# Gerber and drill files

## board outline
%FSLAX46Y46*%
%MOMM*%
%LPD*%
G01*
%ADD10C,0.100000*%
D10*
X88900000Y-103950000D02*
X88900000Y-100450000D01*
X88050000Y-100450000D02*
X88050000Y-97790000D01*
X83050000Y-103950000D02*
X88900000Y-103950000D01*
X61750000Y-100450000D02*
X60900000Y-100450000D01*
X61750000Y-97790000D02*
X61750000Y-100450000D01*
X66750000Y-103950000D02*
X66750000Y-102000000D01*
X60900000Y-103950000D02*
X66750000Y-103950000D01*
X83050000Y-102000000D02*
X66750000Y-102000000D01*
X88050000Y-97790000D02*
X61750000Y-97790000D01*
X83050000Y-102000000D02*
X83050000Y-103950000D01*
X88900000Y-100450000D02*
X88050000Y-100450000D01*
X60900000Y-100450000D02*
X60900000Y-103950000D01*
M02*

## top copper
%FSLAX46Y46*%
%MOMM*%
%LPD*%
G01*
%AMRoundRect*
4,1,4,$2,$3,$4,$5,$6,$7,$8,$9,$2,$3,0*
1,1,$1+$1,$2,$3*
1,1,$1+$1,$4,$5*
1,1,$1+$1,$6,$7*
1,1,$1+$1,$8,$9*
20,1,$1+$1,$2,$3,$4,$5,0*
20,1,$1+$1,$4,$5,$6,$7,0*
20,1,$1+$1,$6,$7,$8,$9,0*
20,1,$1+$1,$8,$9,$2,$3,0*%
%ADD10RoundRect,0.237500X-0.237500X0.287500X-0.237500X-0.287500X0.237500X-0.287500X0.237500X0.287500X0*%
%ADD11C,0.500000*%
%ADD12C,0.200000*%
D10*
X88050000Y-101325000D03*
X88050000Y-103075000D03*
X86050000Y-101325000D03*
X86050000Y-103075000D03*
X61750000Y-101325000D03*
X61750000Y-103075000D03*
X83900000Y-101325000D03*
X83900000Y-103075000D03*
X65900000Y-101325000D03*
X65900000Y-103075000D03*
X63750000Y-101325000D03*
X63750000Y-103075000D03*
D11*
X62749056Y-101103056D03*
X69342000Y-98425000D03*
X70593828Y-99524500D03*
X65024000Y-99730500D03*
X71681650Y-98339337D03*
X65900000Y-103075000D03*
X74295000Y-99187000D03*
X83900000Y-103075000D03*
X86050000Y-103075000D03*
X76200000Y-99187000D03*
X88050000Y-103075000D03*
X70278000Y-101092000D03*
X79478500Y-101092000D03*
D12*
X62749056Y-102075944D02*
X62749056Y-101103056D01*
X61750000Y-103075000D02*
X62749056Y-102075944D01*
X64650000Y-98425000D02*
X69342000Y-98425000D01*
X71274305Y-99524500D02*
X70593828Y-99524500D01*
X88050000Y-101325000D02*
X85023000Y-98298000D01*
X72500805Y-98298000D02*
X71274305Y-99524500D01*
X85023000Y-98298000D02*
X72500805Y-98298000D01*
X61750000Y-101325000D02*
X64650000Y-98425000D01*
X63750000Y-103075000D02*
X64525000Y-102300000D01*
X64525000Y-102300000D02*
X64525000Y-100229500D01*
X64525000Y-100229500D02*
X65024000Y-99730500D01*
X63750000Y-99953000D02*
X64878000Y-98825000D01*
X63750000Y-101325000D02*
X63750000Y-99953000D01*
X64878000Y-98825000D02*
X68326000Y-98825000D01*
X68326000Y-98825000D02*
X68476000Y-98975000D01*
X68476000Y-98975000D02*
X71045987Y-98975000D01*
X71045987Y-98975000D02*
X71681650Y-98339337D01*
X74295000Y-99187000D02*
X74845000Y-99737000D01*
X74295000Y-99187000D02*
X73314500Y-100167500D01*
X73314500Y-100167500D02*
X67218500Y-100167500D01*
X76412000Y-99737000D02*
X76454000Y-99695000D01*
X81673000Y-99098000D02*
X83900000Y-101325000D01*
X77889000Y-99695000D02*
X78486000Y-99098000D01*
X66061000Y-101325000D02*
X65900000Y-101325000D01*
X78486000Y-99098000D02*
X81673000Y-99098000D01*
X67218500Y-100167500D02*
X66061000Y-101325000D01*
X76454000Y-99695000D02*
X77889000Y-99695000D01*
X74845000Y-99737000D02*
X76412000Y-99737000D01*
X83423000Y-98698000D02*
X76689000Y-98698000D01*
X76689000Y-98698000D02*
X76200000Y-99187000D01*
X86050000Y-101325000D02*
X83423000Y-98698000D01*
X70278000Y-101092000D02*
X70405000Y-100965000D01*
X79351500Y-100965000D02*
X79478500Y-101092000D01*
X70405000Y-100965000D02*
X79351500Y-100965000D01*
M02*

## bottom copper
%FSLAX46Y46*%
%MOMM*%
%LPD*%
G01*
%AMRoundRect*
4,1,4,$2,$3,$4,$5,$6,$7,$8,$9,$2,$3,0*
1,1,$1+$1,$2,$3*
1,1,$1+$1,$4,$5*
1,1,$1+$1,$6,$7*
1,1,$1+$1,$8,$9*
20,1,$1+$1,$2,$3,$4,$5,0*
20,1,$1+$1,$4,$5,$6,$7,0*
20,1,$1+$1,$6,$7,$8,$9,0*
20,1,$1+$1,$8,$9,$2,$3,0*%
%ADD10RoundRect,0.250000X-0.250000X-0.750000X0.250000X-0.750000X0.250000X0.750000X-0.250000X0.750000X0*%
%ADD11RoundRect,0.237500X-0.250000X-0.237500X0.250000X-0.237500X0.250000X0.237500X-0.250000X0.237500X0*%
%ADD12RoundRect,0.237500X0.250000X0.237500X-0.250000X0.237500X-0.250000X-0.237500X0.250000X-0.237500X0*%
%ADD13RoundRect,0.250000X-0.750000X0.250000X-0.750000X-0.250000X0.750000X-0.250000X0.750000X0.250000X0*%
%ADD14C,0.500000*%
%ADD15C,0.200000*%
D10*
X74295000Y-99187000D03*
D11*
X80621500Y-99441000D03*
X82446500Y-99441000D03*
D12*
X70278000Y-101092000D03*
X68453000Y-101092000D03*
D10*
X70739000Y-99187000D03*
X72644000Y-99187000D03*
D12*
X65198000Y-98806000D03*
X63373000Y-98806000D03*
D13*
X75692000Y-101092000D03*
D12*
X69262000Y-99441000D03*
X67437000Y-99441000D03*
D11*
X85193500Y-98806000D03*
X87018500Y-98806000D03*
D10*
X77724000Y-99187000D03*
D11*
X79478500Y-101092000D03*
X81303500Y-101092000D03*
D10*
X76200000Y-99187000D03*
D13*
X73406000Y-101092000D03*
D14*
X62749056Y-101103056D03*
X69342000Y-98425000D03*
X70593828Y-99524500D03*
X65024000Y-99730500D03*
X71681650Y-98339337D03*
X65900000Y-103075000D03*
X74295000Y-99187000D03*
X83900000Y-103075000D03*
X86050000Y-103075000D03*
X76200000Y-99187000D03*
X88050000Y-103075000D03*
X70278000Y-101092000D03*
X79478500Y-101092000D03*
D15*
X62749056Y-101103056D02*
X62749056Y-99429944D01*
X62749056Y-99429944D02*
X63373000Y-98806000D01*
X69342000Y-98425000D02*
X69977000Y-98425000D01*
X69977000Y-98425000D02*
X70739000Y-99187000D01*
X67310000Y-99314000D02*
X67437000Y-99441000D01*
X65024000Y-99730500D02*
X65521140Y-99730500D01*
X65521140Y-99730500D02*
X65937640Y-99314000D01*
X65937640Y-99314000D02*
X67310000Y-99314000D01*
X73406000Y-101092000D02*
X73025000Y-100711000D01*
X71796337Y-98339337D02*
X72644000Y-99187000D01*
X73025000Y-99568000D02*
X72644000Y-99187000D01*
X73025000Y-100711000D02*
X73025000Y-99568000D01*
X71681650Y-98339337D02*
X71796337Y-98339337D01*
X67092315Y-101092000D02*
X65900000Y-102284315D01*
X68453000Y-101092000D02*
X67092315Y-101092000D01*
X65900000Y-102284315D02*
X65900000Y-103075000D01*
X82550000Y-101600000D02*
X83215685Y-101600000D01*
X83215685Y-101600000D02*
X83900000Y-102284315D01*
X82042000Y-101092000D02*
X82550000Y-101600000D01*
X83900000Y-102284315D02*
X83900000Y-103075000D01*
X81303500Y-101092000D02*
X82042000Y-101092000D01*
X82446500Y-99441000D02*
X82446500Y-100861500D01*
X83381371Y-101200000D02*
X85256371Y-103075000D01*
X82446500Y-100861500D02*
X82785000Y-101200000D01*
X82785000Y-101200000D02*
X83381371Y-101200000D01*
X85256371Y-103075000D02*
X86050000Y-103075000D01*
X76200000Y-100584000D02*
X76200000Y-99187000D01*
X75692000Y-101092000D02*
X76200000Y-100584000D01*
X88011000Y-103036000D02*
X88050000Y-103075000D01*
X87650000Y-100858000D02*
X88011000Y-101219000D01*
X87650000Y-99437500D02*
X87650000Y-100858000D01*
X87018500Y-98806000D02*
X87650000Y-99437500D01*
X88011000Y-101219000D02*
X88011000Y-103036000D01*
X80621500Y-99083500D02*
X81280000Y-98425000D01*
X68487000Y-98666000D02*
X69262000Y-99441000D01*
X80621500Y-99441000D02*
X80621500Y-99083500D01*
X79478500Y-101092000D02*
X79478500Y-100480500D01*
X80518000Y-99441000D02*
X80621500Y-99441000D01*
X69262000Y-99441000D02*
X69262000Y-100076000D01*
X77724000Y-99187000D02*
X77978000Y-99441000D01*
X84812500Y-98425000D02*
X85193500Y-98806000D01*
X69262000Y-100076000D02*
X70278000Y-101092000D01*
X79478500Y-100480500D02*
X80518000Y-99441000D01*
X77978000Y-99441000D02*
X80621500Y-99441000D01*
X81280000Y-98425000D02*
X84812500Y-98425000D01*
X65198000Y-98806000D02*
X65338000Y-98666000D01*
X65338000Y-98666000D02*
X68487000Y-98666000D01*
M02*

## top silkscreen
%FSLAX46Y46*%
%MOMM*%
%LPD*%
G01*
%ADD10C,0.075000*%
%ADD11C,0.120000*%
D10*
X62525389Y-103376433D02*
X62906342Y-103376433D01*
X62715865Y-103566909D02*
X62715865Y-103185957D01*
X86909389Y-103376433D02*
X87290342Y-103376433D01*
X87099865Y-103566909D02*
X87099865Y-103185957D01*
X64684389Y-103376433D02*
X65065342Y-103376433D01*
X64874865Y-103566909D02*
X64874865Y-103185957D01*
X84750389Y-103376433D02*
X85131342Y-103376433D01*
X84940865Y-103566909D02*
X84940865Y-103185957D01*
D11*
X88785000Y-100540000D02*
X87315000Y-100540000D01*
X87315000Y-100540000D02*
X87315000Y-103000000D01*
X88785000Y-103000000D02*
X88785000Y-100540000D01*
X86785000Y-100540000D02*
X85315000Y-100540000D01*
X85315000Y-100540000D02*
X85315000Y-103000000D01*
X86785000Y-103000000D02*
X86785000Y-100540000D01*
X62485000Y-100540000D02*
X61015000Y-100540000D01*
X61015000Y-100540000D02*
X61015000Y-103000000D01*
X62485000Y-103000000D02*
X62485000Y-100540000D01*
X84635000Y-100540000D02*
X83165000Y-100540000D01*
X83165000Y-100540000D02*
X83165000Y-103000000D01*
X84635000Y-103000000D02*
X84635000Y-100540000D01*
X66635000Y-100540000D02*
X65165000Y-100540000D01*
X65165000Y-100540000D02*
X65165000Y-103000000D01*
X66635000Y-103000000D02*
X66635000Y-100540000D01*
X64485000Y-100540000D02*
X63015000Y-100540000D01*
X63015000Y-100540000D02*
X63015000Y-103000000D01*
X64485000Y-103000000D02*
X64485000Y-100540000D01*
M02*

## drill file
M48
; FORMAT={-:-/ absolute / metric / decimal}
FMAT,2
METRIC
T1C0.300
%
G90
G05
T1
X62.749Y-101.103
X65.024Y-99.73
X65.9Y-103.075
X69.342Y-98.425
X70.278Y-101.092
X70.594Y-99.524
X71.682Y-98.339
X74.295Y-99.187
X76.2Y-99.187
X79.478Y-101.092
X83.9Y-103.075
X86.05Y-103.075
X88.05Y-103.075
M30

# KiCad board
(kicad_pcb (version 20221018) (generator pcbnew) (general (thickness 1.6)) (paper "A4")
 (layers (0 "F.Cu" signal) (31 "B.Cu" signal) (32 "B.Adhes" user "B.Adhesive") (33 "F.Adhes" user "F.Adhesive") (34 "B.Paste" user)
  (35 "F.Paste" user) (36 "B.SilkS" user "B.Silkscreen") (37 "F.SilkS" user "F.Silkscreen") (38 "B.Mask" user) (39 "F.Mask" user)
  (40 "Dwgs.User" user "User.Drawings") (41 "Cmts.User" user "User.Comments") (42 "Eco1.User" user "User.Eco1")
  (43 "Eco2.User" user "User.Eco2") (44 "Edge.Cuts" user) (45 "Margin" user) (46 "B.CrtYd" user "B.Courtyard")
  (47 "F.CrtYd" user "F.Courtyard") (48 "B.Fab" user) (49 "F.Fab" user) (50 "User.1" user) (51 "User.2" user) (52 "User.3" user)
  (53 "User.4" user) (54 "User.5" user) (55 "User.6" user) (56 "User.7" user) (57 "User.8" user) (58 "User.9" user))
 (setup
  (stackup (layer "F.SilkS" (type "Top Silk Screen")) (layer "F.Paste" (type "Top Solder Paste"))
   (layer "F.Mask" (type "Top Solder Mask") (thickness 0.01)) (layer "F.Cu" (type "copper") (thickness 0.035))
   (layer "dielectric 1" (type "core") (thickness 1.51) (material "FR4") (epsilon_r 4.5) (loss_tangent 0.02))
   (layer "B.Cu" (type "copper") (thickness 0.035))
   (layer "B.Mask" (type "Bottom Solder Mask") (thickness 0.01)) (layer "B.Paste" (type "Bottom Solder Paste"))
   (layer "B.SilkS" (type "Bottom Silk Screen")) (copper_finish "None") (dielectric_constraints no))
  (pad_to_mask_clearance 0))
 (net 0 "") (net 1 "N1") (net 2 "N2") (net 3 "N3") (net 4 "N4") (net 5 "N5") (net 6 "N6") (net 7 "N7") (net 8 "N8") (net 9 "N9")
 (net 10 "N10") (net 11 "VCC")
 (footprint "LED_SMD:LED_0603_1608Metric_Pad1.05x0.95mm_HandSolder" (layer "F.Cu") (at 88.05 102.2 -90)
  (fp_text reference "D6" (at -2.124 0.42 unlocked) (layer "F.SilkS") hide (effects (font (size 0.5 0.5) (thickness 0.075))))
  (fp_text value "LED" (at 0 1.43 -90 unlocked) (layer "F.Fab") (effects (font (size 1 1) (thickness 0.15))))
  (fp_line (start -1.66 -0.735) (end -1.66 0.735) (stroke (width 0.12) (type solid)) (layer "F.SilkS"))
  (fp_line (start -1.66 0.735) (end 0.8 0.735) (stroke (width 0.12) (type solid)) (layer "F.SilkS"))
  (fp_line (start 0.8 -0.735) (end -1.66 -0.735) (stroke (width 0.12) (type solid)) (layer "F.SilkS"))
  (pad "1" smd roundrect (at -0.875 0 270) (size 1.05 0.95) (layers "F.Cu" "F.Paste" "F.Mask") (roundrect_rratio 0.25) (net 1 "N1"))
  (pad "2" smd roundrect (at 0.875 0 270) (size 1.05 0.95) (layers "F.Cu" "F.Paste" "F.Mask") (roundrect_rratio 0.25) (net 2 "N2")))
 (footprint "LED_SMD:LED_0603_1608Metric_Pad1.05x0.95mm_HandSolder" (layer "F.Cu") (at 86.05 102.2 -90)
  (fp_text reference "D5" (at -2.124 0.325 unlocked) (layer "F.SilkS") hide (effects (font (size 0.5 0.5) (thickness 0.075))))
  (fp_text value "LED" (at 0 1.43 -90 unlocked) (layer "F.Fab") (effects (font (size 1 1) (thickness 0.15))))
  (fp_line (start -1.66 -0.735) (end -1.66 0.735) (stroke (width 0.12) (type solid)) (layer "F.SilkS"))
  (fp_line (start -1.66 0.735) (end 0.8 0.735) (stroke (width 0.12) (type solid)) (layer "F.SilkS"))
  (fp_line (start 0.8 -0.735) (end -1.66 -0.735) (stroke (width 0.12) (type solid)) (layer "F.SilkS"))
  (pad "1" smd roundrect (at -0.875 0 270) (size 1.05 0.95) (layers "F.Cu" "F.Paste" "F.Mask") (roundrect_rratio 0.25) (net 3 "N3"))
  (pad "2" smd roundrect (at 0.875 0 270) (size 1.05 0.95) (layers "F.Cu" "F.Paste" "F.Mask") (roundrect_rratio 0.25) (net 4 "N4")))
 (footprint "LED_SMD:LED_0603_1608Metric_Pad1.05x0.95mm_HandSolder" (layer "F.Cu") (at 61.75 102.2 -90)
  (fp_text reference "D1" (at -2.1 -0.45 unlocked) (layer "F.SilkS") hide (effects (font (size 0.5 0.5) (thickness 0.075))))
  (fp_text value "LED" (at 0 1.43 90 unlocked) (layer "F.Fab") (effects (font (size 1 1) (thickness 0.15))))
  (fp_line (start -1.66 -0.735) (end -1.66 0.735) (stroke (width 0.12) (type solid)) (layer "F.SilkS"))
  (fp_line (start -1.66 0.735) (end 0.8 0.735) (stroke (width 0.12) (type solid)) (layer "F.SilkS"))
  (fp_line (start 0.8 -0.735) (end -1.66 -0.735) (stroke (width 0.12) (type solid)) (layer "F.SilkS"))
  (pad "1" smd roundrect (at -0.875 0 270) (size 1.05 0.95) (layers "F.Cu" "F.Paste" "F.Mask") (roundrect_rratio 0.25) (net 1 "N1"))
  (pad "2" smd roundrect (at 0.875 0 270) (size 1.05 0.95) (layers "F.Cu" "F.Paste" "F.Mask") (roundrect_rratio 0.25) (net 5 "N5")))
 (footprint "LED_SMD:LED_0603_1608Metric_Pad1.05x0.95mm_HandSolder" (layer "F.Cu") (at 83.9 102.2 -90)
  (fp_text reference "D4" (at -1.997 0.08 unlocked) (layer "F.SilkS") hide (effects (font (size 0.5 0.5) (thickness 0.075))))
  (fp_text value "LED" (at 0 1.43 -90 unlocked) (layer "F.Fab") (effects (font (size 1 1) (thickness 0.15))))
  (fp_line (start -1.66 -0.735) (end -1.66 0.735) (stroke (width 0.12) (type solid)) (layer "F.SilkS"))
  (fp_line (start -1.66 0.735) (end 0.8 0.735) (stroke (width 0.12) (type solid)) (layer "F.SilkS"))
  (fp_line (start 0.8 -0.735) (end -1.66 -0.735) (stroke (width 0.12) (type solid)) (layer "F.SilkS"))
  (pad "1" smd roundrect (at -0.875 0 270) (size 1.05 0.95) (layers "F.Cu" "F.Paste" "F.Mask") (roundrect_rratio 0.25) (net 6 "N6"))
  (pad "2" smd roundrect (at 0.875 0 270) (size 1.05 0.95) (layers "F.Cu" "F.Paste" "F.Mask") (roundrect_rratio 0.25) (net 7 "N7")))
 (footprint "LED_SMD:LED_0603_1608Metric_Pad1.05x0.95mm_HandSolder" (layer "F.Cu") (at 65.9 102.2 -90)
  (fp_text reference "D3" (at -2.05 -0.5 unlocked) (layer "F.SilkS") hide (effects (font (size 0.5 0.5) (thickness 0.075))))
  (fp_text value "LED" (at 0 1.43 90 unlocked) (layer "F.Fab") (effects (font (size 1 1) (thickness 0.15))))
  (fp_line (start -1.66 -0.735) (end -1.66 0.735) (stroke (width 0.12) (type solid)) (layer "F.SilkS"))
  (fp_line (start -1.66 0.735) (end 0.8 0.735) (stroke (width 0.12) (type solid)) (layer "F.SilkS"))
  (fp_line (start 0.8 -0.735) (end -1.66 -0.735) (stroke (width 0.12) (type solid)) (layer "F.SilkS"))
  (pad "1" smd roundrect (at -0.875 0 270) (size 1.05 0.95) (layers "F.Cu" "F.Paste" "F.Mask") (roundrect_rratio 0.25) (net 6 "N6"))
  (pad "2" smd roundrect (at 0.875 0 270) (size 1.05 0.95) (layers "F.Cu" "F.Paste" "F.Mask") (roundrect_rratio 0.25) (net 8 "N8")))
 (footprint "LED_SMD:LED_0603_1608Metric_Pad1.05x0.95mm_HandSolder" (layer "F.Cu") (at 63.75 102.2 -90)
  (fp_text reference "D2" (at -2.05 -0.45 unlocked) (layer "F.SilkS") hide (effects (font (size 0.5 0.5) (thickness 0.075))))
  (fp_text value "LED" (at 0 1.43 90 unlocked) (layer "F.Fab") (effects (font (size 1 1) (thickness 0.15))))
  (fp_line (start -1.66 -0.735) (end -1.66 0.735) (stroke (width 0.12) (type solid)) (layer "F.SilkS"))
  (fp_line (start -1.66 0.735) (end 0.8 0.735) (stroke (width 0.12) (type solid)) (layer "F.SilkS"))
  (fp_line (start 0.8 -0.735) (end -1.66 -0.735) (stroke (width 0.12) (type solid)) (layer "F.SilkS"))
  (pad "1" smd roundrect (at -0.875 0 270) (size 1.05 0.95) (layers "F.Cu" "F.Paste" "F.Mask") (roundrect_rratio 0.25) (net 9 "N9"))
  (pad "2" smd roundrect (at 0.875 0 270) (size 1.05 0.95) (layers "F.Cu" "F.Paste" "F.Mask") (roundrect_rratio 0.25) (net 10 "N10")))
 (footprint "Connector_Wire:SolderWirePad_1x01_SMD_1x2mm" (layer "B.Cu") (at 74.295 99.187)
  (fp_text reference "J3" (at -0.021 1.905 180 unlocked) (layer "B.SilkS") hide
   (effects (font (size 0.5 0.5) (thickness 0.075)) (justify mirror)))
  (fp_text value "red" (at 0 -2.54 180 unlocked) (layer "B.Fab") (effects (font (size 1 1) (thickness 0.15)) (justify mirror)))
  (pad "1" smd roundrect (at 0 0) (size 1 2) (layers "B.Cu" "B.Paste" "B.Mask") (roundrect_rratio 0.25) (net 6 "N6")))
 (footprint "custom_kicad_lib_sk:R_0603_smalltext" (layer "B.Cu") (at 81.534 99.441)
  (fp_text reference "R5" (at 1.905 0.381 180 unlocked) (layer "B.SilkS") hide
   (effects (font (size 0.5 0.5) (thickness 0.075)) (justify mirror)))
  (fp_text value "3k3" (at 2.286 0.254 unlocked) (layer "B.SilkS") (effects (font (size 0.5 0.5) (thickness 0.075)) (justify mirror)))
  (pad "1" smd roundrect (at -0.9125 0) (size 0.975 0.95) (layers "B.Cu" "B.Paste" "B.Mask") (roundrect_rratio 0.25) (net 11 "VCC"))
  (pad "2" smd roundrect (at 0.9125 0) (size 0.975 0.95) (layers "B.Cu" "B.Paste" "B.Mask") (roundrect_rratio 0.25) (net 4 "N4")))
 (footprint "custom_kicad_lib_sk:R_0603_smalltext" (layer "B.Cu") (at 69.3655 101.092 180)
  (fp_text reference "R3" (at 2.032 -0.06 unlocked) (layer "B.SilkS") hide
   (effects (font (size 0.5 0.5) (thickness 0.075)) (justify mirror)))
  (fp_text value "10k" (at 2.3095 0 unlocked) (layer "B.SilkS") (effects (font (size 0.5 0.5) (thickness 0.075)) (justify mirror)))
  (pad "1" smd roundrect (at -0.9125 0 180) (size 0.975 0.95) (layers "B.Cu" "B.Paste" "B.Mask") (roundrect_rratio 0.25) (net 11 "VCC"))
  (pad "2" smd roundrect (at 0.9125 0 180) (size 0.975 0.95) (layers "B.Cu" "B.Paste" "B.Mask") (roundrect_rratio 0.25) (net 8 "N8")))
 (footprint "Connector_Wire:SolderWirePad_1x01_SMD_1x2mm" (layer "B.Cu") (at 70.739 99.187)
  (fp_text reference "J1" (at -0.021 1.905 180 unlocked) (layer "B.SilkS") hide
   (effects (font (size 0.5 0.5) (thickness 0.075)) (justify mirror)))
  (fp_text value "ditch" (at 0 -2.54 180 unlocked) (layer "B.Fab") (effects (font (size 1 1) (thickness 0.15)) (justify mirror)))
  (pad "1" smd roundrect (at 0 0) (size 1 2) (layers "B.Cu" "B.Paste" "B.Mask") (roundrect_rratio 0.25) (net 1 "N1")))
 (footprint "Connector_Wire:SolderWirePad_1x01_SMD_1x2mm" (layer "B.Cu") (at 72.644 99.187)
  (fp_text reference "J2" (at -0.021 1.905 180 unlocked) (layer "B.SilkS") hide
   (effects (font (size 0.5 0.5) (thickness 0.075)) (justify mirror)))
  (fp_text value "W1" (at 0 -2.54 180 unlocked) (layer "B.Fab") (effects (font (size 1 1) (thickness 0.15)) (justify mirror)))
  (pad "1" smd roundrect (at 0 0) (size 1 2) (layers "B.Cu" "B.Paste" "B.Mask") (roundrect_rratio 0.25) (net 9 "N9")))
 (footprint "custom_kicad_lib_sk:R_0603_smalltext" (layer "B.Cu") (at 64.2855 98.806 180)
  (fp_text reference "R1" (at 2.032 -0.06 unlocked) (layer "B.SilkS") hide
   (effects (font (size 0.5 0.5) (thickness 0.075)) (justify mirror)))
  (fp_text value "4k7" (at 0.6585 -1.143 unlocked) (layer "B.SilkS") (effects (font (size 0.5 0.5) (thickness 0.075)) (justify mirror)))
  (pad "1" smd roundrect (at -0.9125 0 180) (size 0.975 0.95) (layers "B.Cu" "B.Paste" "B.Mask") (roundrect_rratio 0.25) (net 11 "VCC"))
  (pad "2" smd roundrect (at 0.9125 0 180) (size 0.975 0.95) (layers "B.Cu" "B.Paste" "B.Mask") (roundrect_rratio 0.25) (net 5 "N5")))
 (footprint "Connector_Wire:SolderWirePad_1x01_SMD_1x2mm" (layer "B.Cu") (at 75.692 101.092 -90)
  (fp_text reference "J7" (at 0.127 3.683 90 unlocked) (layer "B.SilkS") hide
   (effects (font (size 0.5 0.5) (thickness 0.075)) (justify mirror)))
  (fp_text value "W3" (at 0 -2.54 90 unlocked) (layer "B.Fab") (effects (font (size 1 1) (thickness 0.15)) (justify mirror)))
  (pad "1" smd roundrect (at 0 0 270) (size 1 2) (layers "B.Cu" "B.Paste" "B.Mask") (roundrect_rratio 0.25) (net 3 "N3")))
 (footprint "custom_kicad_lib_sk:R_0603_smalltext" (layer "B.Cu") (at 68.3495 99.441 180)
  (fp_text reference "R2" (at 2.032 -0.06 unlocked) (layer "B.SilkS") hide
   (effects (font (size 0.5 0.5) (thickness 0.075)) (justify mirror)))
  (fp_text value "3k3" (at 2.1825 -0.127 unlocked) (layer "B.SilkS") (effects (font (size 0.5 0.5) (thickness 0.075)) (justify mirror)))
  (pad "1" smd roundrect (at -0.9125 0 180) (size 0.975 0.95) (layers "B.Cu" "B.Paste" "B.Mask") (roundrect_rratio 0.25) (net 11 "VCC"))
  (pad "2" smd roundrect (at 0.9125 0 180) (size 0.975 0.95) (layers "B.Cu" "B.Paste" "B.Mask") (roundrect_rratio 0.25) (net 10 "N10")))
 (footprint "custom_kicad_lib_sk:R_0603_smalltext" (layer "B.Cu") (at 86.106 98.806)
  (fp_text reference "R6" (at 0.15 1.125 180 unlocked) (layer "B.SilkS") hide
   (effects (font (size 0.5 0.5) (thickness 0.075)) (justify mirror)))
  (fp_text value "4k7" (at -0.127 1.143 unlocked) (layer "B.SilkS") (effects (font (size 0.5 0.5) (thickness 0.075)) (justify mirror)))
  (pad "1" smd roundrect (at -0.9125 0) (size 0.975 0.95) (layers "B.Cu" "B.Paste" "B.Mask") (roundrect_rratio 0.25) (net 11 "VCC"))
  (pad "2" smd roundrect (at 0.9125 0) (size 0.975 0.95) (layers "B.Cu" "B.Paste" "B.Mask") (roundrect_rratio 0.25) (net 2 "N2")))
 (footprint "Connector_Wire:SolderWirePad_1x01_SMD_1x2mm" (layer "B.Cu") (at 77.724 99.187)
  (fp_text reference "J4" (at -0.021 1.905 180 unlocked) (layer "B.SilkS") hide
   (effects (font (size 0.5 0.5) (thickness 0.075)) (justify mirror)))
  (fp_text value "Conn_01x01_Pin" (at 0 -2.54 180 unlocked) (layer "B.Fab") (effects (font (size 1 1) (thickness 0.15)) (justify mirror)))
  (pad "1" smd roundrect (at 0 0) (size 1 2) (layers "B.Cu" "B.Paste" "B.Mask") (roundrect_rratio 0.25) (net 11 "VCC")))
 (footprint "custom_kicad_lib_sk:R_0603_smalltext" (layer "B.Cu") (at 80.391 101.092)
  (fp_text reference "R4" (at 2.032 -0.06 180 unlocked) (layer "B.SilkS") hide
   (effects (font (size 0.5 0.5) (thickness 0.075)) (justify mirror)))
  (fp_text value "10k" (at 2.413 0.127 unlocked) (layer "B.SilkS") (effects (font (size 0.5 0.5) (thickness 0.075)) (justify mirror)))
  (pad "1" smd roundrect (at -0.9125 0) (size 0.975 0.95) (layers "B.Cu" "B.Paste" "B.Mask") (roundrect_rratio 0.25) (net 11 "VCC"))
  (pad "2" smd roundrect (at 0.9125 0) (size 0.975 0.95) (layers "B.Cu" "B.Paste" "B.Mask") (roundrect_rratio 0.25) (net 7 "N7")))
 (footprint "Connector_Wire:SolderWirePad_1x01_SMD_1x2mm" (layer "B.Cu") (at 76.2 99.187)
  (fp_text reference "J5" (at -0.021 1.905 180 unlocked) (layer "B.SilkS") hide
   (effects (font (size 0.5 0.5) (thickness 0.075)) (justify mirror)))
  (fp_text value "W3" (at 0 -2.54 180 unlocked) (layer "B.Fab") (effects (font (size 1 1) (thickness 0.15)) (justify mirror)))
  (pad "1" smd roundrect (at 0 0) (size 1 2) (layers "B.Cu" "B.Paste" "B.Mask") (roundrect_rratio 0.25) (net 3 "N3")))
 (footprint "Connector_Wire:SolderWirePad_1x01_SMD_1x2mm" (layer "B.Cu") (at 73.406 101.092 -90)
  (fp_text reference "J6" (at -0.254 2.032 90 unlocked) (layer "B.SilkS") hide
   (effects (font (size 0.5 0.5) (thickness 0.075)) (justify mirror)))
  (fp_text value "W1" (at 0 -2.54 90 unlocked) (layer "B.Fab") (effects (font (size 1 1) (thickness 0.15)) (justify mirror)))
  (pad "1" smd roundrect (at 0 0 270) (size 1 2) (layers "B.Cu" "B.Paste" "B.Mask") (roundrect_rratio 0.25) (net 9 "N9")))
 (gr_line (start 88.9 103.95) (end 88.9 100.45) (stroke (width 0.1) (type default)) (layer "Edge.Cuts"))
 (gr_line (start 88.05 100.45) (end 88.05 97.79) (stroke (width 0.1) (type default)) (layer "Edge.Cuts"))
 (gr_line (start 83.05 103.95) (end 88.9 103.95) (stroke (width 0.1) (type default)) (layer "Edge.Cuts"))
 (gr_line (start 61.75 100.45) (end 60.9 100.45) (stroke (width 0.1) (type default)) (layer "Edge.Cuts"))
 (gr_line (start 61.75 97.79) (end 61.75 100.45) (stroke (width 0.1) (type default)) (layer "Edge.Cuts"))
 (gr_line (start 66.75 103.95) (end 66.75 102) (stroke (width 0.1) (type default)) (layer "Edge.Cuts"))
 (gr_line (start 60.9 103.95) (end 66.75 103.95) (stroke (width 0.1) (type default)) (layer "Edge.Cuts"))
 (gr_line (start 83.05 102) (end 66.75 102) (stroke (width 0.1) (type default)) (layer "Edge.Cuts"))
 (gr_line (start 88.05 97.79) (end 61.75 97.79) (stroke (width 0.1) (type default)) (layer "Edge.Cuts"))
 (gr_line (start 83.05 102) (end 83.05 103.95) (stroke (width 0.1) (type default)) (layer "Edge.Cuts"))
 (gr_line (start 88.9 100.45) (end 88.05 100.45) (stroke (width 0.1) (type default)) (layer "Edge.Cuts"))
 (gr_line (start 60.9 100.45) (end 60.9 103.95) (stroke (width 0.1) (type default)) (layer "Edge.Cuts"))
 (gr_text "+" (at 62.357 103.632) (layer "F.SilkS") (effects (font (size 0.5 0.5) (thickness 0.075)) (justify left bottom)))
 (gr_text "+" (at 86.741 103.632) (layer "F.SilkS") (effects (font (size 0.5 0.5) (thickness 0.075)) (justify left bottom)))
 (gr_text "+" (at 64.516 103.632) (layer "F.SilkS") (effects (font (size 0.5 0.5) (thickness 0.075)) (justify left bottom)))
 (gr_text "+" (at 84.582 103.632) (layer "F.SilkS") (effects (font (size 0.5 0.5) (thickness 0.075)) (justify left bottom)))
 (segment (start 62.749056 102.075944) (end 62.749056 101.103056) (width 0.2) (layer "F.Cu") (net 5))
 (segment (start 61.75 103.075) (end 62.749056 102.075944) (width 0.2) (layer "F.Cu") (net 5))
 (via (at 62.749056 101.103056) (size 0.5) (drill 0.3) (layers "F.Cu" "B.Cu") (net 5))
 (segment (start 62.749056 101.103056) (end 62.749056 99.429944) (width 0.2) (layer "B.Cu") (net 5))
 (segment (start 62.749056 99.429944) (end 63.373 98.806) (width 0.2) (layer "B.Cu") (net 5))
 (segment (start 64.65 98.425) (end 69.342 98.425) (width 0.2) (layer "F.Cu") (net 1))
 (segment (start 71.274305 99.5245) (end 70.593828 99.5245) (width 0.2) (layer "F.Cu") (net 1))
 (segment (start 88.05 101.325) (end 85.023 98.298) (width 0.2) (layer "F.Cu") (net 1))
 (segment (start 72.500805 98.298) (end 71.274305 99.5245) (width 0.2) (layer "F.Cu") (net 1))
 (segment (start 85.023 98.298) (end 72.500805 98.298) (width 0.2) (layer "F.Cu") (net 1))
 (segment (start 61.75 101.325) (end 64.65 98.425) (width 0.2) (layer "F.Cu") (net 1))
 (via (at 69.342 98.425) (size 0.5) (drill 0.3) (layers "F.Cu" "B.Cu") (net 1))
 (via (at 70.593828 99.5245) (size 0.5) (drill 0.3) (layers "F.Cu" "B.Cu") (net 1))
 (segment (start 69.342 98.425) (end 69.977 98.425) (width 0.2) (layer "B.Cu") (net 1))
 (segment (start 69.977 98.425) (end 70.739 99.187) (width 0.2) (layer "B.Cu") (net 1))
 (segment (start 63.75 103.075) (end 64.525 102.3) (width 0.2) (layer "F.Cu") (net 10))
 (segment (start 64.525 102.3) (end 64.525 100.2295) (width 0.2) (layer "F.Cu") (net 10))
 (segment (start 64.525 100.2295) (end 65.024 99.7305) (width 0.2) (layer "F.Cu") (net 10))
 (via (at 65.024 99.7305) (size 0.5) (drill 0.3) (layers "F.Cu" "B.Cu") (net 10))
 (segment (start 67.31 99.314) (end 67.437 99.441) (width 0.2) (layer "B.Cu") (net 10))
 (segment (start 65.024 99.7305) (end 65.52114 99.7305) (width 0.2) (layer "B.Cu") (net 10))
 (segment (start 65.52114 99.7305) (end 65.93764 99.314) (width 0.2) (layer "B.Cu") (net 10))
 (segment (start 65.93764 99.314) (end 67.31 99.314) (width 0.2) (layer "B.Cu") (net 10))
 (segment (start 63.75 99.953) (end 64.878 98.825) (width 0.2) (layer "F.Cu") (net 9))
 (segment (start 63.75 101.325) (end 63.75 99.953) (width 0.2) (layer "F.Cu") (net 9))
 (segment (start 64.878 98.825) (end 68.326 98.825) (width 0.2) (layer "F.Cu") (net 9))
 (segment (start 68.326 98.825) (end 68.476 98.975) (width 0.2) (layer "F.Cu") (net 9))
 (segment (start 68.476 98.975) (end 71.045987 98.975) (width 0.2) (layer "F.Cu") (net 9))
 (segment (start 71.045987 98.975) (end 71.68165 98.339337) (width 0.2) (layer "F.Cu") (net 9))
 (via (at 71.68165 98.339337) (size 0.5) (drill 0.3) (layers "F.Cu" "B.Cu") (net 9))
 (segment (start 73.406 101.092) (end 73.025 100.711) (width 0.2) (layer "B.Cu") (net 9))
 (segment (start 71.796337 98.339337) (end 72.644 99.187) (width 0.2) (layer "B.Cu") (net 9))
 (segment (start 73.025 99.568) (end 72.644 99.187) (width 0.2) (layer "B.Cu") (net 9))
 (segment (start 73.025 100.711) (end 73.025 99.568) (width 0.2) (layer "B.Cu") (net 9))
 (segment (start 71.68165 98.339337) (end 71.796337 98.339337) (width 0.2) (layer "B.Cu") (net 9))
 (via (at 65.9 103.075) (size 0.5) (drill 0.3) (layers "F.Cu" "B.Cu") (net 8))
 (segment (start 67.092315 101.092) (end 65.9 102.284315) (width 0.2) (layer "B.Cu") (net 8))
 (segment (start 68.453 101.092) (end 67.092315 101.092) (width 0.2) (layer "B.Cu") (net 8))
 (segment (start 65.9 102.284315) (end 65.9 103.075) (width 0.2) (layer "B.Cu") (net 8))
 (segment (start 74.295 99.187) (end 74.845 99.737) (width 0.2) (layer "F.Cu") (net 6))
 (segment (start 74.295 99.187) (end 73.3145 100.1675) (width 0.2) (layer "F.Cu") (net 6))
 (segment (start 73.3145 100.1675) (end 67.2185 100.1675) (width 0.2) (layer "F.Cu") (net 6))
 (segment (start 76.412 99.737) (end 76.454 99.695) (width 0.2) (layer "F.Cu") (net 6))
 (segment (start 81.673 99.098) (end 83.9 101.325) (width 0.2) (layer "F.Cu") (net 6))
 (segment (start 77.889 99.695) (end 78.486 99.098) (width 0.2) (layer "F.Cu") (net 6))
 (segment (start 66.061 101.325) (end 65.9 101.325) (width 0.2) (layer "F.Cu") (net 6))
 (segment (start 78.486 99.098) (end 81.673 99.098) (width 0.2) (layer "F.Cu") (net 6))
 (segment (start 67.2185 100.1675) (end 66.061 101.325) (width 0.2) (layer "F.Cu") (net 6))
 (segment (start 76.454 99.695) (end 77.889 99.695) (width 0.2) (layer "F.Cu") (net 6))
 (segment (start 74.845 99.737) (end 76.412 99.737) (width 0.2) (layer "F.Cu") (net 6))
 (via (at 74.295 99.187) (size 0.5) (drill 0.3) (layers "F.Cu" "B.Cu") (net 6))
 (via (at 83.9 103.075) (size 0.5) (drill 0.3) (layers "F.Cu" "B.Cu") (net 7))
 (segment (start 82.55 101.6) (end 83.215685 101.6) (width 0.2) (layer "B.Cu") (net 7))
 (segment (start 83.215685 101.6) (end 83.9 102.284315) (width 0.2) (layer "B.Cu") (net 7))
 (segment (start 82.042 101.092) (end 82.55 101.6) (width 0.2) (layer "B.Cu") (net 7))
 (segment (start 83.9 102.284315) (end 83.9 103.075) (width 0.2) (layer "B.Cu") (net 7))
 (segment (start 81.3035 101.092) (end 82.042 101.092) (width 0.2) (layer "B.Cu") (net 7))
 (via (at 86.05 103.075) (size 0.5) (drill 0.3) (layers "F.Cu" "B.Cu") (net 4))
 (segment (start 82.4465 99.441) (end 82.4465 100.8615) (width 0.2) (layer "B.Cu") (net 4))
 (segment (start 83.381371 101.2) (end 85.256371 103.075) (width 0.2) (layer "B.Cu") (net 4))
 (segment (start 82.4465 100.8615) (end 82.785 101.2) (width 0.2) (layer "B.Cu") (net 4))
 (segment (start 82.785 101.2) (end 83.381371 101.2) (width 0.2) (layer "B.Cu") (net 4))
 (segment (start 85.256371 103.075) (end 86.05 103.075) (width 0.2) (layer "B.Cu") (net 4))
 (segment (start 83.423 98.698) (end 76.689 98.698) (width 0.2) (layer "F.Cu") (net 3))
 (segment (start 76.689 98.698) (end 76.2 99.187) (width 0.2) (layer "F.Cu") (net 3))
 (segment (start 86.05 101.325) (end 83.423 98.698) (width 0.2) (layer "F.Cu") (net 3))
 (via (at 76.2 99.187) (size 0.5) (drill 0.3) (layers "F.Cu" "B.Cu") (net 3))
 (segment (start 76.2 100.584) (end 76.2 99.187) (width 0.2) (layer "B.Cu") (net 3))
 (segment (start 75.692 101.092) (end 76.2 100.584) (width 0.2) (layer "B.Cu") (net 3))
 (via (at 88.05 103.075) (size 0.5) (drill 0.3) (layers "F.Cu" "B.Cu") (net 2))
 (segment (start 88.011 103.036) (end 88.05 103.075) (width 0.2) (layer "B.Cu") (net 2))
 (segment (start 87.65 100.858) (end 88.011 101.219) (width 0.2) (layer "B.Cu") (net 2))
 (segment (start 87.65 99.4375) (end 87.65 100.858) (width 0.2) (layer "B.Cu") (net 2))
 (segment (start 87.0185 98.806) (end 87.65 99.4375) (width 0.2) (layer "B.Cu") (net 2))
 (segment (start 88.011 101.219) (end 88.011 103.036) (width 0.2) (layer "B.Cu") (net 2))
 (segment (start 70.278 101.092) (end 70.405 100.965) (width 0.2) (layer "F.Cu") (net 11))
 (segment (start 79.3515 100.965) (end 79.4785 101.092) (width 0.2) (layer "F.Cu") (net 11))
 (segment (start 70.405 100.965) (end 79.3515 100.965) (width 0.2) (layer "F.Cu") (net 11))
 (via (at 70.278 101.092) (size 0.5) (drill 0.3) (layers "F.Cu" "B.Cu") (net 11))
 (via (at 79.4785 101.092) (size 0.5) (drill 0.3) (layers "F.Cu" "B.Cu") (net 11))
 (segment (start 80.6215 99.0835) (end 81.28 98.425) (width 0.2) (layer "B.Cu") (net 11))
 (segment (start 68.487 98.666) (end 69.262 99.441) (width 0.2) (layer "B.Cu") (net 11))
 (segment (start 80.6215 99.441) (end 80.6215 99.0835) (width 0.2) (layer "B.Cu") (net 11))
 (segment (start 79.4785 101.092) (end 79.4785 100.4805) (width 0.2) (layer "B.Cu") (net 11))
 (segment (start 80.518 99.441) (end 80.6215 99.441) (width 0.2) (layer "B.Cu") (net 11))
 (segment (start 69.262 99.441) (end 69.262 100.076) (width 0.2) (layer "B.Cu") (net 11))
 (segment (start 77.724 99.187) (end 77.978 99.441) (width 0.2) (layer "B.Cu") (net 11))
 (segment (start 84.8125 98.425) (end 85.1935 98.806) (width 0.2) (layer "B.Cu") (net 11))
 (segment (start 69.262 100.076) (end 70.278 101.092) (width 0.2) (layer "B.Cu") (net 11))
 (segment (start 79.4785 100.4805) (end 80.518 99.441) (width 0.2) (layer "B.Cu") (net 11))
 (segment (start 77.978 99.441) (end 80.6215 99.441) (width 0.2) (layer "B.Cu") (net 11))
 (segment (start 81.28 98.425) (end 84.8125 98.425) (width 0.2) (layer "B.Cu") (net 11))
 (segment (start 65.198 98.806) (end 65.338 98.666) (width 0.2) (layer "B.Cu") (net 11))
 (segment (start 65.338 98.666) (end 68.487 98.666) (width 0.2) (layer "B.Cu") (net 11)))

